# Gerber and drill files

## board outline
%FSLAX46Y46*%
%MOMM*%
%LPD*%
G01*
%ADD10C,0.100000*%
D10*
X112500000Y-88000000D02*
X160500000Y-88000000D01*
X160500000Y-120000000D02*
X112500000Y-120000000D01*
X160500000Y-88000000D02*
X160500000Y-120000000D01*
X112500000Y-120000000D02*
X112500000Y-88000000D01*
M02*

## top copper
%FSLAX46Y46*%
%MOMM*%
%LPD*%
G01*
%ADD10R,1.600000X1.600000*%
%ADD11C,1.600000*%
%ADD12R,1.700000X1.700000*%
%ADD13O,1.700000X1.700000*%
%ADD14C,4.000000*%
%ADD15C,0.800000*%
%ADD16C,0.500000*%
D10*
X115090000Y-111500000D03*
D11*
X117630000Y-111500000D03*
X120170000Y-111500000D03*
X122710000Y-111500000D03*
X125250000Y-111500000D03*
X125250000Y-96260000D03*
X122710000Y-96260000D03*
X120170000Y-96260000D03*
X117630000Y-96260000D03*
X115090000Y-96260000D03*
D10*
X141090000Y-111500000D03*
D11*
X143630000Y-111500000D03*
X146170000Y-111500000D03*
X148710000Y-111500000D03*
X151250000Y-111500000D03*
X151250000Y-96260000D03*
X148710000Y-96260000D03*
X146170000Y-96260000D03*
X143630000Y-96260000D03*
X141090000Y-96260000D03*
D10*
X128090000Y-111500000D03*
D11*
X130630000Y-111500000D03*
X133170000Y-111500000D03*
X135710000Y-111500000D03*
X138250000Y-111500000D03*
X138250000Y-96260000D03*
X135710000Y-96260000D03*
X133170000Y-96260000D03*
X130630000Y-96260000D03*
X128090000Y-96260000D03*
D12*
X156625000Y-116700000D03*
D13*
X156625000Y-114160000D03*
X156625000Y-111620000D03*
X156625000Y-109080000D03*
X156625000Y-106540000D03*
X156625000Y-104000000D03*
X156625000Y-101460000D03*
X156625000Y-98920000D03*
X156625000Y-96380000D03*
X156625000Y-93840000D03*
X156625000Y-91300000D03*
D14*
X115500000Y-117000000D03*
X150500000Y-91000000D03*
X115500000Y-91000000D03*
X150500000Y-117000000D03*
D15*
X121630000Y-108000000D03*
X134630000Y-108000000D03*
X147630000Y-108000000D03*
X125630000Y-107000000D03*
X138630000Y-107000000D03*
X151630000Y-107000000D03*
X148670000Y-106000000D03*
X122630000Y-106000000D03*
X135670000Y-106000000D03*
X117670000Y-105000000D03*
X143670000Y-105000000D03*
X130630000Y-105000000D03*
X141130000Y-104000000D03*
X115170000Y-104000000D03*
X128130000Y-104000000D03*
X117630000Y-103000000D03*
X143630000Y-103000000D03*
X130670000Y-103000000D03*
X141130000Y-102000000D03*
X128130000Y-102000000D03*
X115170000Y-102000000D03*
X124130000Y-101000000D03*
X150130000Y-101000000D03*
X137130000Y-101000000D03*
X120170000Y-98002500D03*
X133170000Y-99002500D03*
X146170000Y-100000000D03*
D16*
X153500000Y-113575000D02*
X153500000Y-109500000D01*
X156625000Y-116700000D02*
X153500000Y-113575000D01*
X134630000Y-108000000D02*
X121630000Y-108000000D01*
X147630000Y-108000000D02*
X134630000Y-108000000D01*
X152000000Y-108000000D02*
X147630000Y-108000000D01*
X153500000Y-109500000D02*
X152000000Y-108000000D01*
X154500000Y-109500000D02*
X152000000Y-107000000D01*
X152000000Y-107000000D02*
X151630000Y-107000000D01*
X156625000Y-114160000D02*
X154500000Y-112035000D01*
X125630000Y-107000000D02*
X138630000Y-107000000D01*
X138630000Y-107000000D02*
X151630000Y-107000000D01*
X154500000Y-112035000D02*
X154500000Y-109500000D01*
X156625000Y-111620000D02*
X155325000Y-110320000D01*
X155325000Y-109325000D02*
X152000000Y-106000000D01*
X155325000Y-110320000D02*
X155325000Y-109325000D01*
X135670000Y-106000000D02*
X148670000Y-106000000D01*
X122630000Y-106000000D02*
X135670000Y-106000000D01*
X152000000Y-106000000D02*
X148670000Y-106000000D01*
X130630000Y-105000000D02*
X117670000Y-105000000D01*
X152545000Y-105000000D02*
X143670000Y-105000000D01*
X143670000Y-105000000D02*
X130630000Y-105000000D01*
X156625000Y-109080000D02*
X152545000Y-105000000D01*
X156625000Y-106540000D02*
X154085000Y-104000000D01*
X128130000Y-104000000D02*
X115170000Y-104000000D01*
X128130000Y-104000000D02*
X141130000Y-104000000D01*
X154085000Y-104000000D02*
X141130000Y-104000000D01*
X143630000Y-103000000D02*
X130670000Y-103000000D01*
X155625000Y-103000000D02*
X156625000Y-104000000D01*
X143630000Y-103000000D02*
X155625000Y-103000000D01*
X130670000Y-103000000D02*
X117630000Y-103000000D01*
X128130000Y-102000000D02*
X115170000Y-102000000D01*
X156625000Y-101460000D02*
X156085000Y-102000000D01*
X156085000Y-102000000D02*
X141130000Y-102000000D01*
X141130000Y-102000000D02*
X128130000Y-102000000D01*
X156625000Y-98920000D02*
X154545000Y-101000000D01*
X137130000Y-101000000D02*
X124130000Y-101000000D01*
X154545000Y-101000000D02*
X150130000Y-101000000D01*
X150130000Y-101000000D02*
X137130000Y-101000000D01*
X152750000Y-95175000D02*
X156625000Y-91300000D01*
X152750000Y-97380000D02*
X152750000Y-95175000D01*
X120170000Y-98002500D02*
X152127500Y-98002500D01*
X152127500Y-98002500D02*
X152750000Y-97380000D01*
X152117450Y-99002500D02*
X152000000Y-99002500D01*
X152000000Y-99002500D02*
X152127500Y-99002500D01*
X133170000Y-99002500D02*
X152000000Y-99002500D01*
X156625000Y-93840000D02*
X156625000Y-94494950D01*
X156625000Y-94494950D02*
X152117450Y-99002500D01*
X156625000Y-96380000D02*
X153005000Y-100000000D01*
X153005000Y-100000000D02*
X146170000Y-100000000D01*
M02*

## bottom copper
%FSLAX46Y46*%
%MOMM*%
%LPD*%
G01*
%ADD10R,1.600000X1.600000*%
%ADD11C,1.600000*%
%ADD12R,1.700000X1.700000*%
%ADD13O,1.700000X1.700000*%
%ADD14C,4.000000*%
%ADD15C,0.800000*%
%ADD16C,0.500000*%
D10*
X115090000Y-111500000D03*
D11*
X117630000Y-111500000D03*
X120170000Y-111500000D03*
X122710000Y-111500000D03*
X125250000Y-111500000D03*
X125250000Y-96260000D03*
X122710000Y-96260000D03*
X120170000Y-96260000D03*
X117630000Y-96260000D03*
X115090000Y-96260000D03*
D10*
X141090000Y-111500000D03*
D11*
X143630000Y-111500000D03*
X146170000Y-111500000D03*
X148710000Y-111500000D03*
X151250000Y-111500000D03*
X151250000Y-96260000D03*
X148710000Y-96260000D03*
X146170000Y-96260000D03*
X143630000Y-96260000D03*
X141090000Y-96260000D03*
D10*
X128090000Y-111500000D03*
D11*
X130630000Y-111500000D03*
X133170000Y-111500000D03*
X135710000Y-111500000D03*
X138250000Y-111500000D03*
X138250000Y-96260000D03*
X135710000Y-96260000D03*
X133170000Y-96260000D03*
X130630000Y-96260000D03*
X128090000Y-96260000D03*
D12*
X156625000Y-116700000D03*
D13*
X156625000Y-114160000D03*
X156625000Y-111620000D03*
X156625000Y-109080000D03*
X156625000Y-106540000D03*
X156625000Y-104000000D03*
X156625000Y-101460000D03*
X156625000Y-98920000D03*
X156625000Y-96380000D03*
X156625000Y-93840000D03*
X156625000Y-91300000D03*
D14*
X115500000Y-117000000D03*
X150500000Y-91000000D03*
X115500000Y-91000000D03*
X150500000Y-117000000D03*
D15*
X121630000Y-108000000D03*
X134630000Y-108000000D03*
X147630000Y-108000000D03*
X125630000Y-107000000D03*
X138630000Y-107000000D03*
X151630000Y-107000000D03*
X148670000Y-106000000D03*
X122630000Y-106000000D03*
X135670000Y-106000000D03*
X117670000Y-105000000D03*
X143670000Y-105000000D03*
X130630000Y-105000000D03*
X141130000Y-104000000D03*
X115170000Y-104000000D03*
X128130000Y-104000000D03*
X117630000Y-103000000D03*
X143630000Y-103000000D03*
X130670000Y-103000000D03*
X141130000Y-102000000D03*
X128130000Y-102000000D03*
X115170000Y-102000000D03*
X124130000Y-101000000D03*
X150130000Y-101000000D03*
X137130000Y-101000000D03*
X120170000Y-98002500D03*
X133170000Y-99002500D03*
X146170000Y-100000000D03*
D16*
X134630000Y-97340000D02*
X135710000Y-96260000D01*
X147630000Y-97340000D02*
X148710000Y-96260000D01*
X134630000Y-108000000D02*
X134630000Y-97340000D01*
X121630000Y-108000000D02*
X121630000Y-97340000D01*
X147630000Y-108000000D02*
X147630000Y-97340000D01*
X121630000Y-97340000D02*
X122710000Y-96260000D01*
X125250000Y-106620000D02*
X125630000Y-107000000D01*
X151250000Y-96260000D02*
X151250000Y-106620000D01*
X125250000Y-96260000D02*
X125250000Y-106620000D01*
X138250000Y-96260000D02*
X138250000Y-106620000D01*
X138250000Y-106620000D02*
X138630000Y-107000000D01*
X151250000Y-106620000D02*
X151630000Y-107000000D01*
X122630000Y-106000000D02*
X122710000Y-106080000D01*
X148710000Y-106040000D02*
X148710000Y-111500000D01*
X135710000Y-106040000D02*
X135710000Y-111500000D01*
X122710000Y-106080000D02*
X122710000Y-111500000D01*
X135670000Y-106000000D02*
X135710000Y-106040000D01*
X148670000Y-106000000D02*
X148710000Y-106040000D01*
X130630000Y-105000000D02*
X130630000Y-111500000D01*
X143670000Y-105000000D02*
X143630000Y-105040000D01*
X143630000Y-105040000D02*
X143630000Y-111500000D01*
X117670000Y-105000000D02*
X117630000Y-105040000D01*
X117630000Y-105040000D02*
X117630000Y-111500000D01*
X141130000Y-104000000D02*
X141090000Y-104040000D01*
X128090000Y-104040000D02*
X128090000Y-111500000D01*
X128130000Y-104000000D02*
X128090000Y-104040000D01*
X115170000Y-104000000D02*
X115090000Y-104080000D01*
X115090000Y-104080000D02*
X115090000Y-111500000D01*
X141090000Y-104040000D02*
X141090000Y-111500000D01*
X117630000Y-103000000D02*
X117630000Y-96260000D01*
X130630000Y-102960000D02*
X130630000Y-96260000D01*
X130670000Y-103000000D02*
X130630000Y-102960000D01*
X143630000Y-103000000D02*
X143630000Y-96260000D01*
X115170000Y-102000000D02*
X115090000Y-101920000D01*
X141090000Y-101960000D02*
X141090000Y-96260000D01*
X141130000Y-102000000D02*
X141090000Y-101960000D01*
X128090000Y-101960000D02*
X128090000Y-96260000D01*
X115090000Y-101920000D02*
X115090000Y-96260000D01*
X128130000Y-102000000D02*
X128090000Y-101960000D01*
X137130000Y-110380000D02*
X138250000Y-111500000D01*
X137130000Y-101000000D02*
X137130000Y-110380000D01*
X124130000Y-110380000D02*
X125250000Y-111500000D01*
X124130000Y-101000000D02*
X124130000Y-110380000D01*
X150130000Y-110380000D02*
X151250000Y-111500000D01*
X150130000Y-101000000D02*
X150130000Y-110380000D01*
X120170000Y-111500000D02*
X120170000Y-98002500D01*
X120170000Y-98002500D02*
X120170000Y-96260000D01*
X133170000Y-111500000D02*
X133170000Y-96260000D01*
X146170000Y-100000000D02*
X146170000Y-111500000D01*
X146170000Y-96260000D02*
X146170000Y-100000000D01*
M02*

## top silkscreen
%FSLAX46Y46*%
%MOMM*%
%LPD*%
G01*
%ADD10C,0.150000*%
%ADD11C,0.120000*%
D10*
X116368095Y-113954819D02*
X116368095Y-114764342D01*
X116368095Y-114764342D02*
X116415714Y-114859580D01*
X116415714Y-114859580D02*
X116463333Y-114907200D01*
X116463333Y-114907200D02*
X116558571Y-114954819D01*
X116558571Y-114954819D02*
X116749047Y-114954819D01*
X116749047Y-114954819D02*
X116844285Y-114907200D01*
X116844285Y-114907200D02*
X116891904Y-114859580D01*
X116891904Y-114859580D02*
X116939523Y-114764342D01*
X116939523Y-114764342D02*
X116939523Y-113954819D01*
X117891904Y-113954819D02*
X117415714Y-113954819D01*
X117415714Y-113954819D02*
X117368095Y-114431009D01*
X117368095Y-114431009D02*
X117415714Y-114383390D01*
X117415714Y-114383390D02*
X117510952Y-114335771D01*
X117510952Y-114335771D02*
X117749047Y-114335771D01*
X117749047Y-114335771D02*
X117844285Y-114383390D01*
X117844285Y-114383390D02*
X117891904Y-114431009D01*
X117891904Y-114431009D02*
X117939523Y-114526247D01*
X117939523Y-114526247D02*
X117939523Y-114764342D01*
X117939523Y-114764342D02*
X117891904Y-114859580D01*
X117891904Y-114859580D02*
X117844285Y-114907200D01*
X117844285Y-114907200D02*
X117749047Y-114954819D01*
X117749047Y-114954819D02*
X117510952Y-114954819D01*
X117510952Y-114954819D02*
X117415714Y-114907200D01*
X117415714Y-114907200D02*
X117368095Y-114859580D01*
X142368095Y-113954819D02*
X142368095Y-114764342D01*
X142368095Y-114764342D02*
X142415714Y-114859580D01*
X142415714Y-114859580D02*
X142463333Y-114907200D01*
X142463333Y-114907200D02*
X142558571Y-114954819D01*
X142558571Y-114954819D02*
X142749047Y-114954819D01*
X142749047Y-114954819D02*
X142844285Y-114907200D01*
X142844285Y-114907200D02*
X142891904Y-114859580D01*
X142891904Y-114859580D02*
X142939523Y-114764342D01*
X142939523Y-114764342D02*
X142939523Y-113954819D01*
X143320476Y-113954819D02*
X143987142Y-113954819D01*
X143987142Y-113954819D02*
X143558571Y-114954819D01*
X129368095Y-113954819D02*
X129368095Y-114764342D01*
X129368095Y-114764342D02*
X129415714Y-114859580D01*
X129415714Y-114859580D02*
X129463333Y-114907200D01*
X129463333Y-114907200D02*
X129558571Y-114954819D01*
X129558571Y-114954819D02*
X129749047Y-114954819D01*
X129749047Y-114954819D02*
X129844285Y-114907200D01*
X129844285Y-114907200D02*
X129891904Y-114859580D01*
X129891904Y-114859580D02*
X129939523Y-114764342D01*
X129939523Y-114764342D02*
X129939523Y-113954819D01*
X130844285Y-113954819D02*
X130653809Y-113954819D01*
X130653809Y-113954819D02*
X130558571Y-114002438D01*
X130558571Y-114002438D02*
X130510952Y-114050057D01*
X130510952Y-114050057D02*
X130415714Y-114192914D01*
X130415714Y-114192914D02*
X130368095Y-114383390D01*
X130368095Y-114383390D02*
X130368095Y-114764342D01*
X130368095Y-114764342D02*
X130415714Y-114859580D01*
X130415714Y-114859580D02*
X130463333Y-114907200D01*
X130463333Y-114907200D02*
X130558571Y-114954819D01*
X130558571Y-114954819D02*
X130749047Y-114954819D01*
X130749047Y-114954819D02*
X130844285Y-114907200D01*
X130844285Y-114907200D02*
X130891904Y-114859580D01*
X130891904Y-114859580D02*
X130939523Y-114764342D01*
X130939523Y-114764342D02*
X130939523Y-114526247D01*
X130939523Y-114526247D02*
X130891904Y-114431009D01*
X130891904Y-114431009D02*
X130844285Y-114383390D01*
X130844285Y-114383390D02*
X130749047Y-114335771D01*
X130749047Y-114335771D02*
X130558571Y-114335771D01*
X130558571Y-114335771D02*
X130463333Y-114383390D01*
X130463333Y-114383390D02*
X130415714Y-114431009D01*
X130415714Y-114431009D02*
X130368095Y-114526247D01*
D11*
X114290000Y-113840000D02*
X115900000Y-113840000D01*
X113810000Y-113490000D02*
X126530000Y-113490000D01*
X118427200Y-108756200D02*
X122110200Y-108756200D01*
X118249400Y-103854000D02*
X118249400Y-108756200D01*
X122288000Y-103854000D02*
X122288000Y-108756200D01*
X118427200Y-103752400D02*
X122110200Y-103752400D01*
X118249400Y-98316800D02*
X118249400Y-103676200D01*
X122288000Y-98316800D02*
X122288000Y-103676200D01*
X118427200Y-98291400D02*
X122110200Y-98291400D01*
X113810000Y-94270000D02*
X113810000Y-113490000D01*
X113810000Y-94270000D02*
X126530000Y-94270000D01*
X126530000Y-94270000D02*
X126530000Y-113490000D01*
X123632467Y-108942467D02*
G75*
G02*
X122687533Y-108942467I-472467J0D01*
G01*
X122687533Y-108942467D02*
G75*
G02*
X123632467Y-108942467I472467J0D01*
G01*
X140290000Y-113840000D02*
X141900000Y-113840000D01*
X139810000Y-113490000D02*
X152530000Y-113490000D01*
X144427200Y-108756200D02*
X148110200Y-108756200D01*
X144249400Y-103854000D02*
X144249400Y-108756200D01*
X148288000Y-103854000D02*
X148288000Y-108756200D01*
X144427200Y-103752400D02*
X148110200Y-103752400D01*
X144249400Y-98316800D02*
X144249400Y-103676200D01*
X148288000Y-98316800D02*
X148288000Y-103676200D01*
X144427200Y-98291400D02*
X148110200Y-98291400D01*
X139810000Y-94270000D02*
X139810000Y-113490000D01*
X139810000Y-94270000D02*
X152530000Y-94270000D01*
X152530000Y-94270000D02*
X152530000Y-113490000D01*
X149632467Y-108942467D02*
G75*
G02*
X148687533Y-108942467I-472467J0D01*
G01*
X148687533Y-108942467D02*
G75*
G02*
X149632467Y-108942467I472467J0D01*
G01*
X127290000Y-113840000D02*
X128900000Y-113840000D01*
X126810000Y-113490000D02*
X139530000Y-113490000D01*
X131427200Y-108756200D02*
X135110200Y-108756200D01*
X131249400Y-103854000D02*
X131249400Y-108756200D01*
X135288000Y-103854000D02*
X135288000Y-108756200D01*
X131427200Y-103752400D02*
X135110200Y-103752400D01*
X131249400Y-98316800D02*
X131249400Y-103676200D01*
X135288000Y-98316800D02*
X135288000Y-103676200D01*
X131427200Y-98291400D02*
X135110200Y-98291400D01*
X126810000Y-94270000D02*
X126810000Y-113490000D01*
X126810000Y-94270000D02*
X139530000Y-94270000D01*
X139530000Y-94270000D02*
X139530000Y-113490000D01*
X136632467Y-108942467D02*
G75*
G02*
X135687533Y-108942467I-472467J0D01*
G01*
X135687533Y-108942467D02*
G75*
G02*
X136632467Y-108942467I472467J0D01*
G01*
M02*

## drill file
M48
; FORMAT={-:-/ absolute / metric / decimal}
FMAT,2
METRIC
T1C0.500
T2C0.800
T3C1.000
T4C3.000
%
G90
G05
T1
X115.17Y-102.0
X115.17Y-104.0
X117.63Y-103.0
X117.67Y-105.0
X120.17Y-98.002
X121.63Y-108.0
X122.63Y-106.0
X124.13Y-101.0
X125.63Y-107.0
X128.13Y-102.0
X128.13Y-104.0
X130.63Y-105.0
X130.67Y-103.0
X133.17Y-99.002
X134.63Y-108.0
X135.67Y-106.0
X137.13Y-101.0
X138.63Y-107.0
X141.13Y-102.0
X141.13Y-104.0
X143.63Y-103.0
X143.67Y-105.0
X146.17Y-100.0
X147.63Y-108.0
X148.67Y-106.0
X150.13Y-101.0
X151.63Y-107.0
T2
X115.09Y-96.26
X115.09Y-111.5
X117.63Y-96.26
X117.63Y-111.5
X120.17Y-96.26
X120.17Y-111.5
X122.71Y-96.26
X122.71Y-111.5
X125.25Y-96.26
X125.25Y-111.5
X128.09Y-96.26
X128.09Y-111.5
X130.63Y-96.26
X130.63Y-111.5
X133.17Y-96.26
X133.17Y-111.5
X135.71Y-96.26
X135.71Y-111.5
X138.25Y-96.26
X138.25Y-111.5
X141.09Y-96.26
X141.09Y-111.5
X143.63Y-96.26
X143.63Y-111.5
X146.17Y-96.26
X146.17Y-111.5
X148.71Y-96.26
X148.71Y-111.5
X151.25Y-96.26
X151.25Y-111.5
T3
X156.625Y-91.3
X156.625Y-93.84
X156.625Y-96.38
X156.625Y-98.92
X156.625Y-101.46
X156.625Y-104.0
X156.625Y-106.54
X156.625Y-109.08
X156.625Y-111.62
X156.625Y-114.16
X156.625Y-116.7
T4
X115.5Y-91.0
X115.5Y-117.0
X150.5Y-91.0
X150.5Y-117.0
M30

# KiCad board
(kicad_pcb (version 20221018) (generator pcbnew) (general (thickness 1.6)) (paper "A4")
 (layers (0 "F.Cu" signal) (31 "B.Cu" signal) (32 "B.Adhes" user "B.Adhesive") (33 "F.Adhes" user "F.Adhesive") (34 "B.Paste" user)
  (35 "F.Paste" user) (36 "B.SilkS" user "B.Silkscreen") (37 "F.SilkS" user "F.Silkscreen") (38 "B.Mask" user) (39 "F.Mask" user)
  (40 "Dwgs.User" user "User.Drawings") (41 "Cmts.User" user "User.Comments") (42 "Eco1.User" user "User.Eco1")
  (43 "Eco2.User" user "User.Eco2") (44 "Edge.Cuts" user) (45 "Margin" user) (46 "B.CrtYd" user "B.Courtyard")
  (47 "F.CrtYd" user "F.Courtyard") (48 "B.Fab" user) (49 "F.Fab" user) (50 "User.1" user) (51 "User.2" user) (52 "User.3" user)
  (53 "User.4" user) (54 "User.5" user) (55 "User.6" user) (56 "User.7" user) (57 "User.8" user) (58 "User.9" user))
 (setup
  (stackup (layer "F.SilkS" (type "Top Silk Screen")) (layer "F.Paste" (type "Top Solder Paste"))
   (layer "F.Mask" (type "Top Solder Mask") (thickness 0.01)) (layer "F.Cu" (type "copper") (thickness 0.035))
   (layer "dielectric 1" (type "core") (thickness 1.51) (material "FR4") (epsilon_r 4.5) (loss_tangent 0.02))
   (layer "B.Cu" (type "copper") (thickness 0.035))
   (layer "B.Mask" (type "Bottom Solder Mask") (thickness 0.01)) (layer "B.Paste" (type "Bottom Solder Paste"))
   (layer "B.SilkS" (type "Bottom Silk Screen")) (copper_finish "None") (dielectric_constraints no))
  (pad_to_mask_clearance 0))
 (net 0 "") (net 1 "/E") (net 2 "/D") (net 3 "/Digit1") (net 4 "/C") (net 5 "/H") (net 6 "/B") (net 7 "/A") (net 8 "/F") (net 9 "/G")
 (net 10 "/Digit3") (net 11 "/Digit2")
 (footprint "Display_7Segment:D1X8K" (layer "F.Cu") (at 115.09 111.5 90)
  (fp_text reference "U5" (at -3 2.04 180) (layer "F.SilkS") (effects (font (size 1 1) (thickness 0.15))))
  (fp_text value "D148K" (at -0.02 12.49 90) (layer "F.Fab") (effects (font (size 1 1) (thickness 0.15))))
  (fp_line (start -2.34 -0.8) (end -2.34 0.81) (stroke (width 0.12) (type solid)) (layer "F.SilkS"))
  (fp_line (start -1.99 -1.28) (end -1.99 11.44) (stroke (width 0.12) (type solid)) (layer "F.SilkS"))
  (fp_line (start 2.7438 3.3372) (end 2.7438 7.0202) (stroke (width 0.12) (type solid)) (layer "F.SilkS"))
  (fp_line (start 7.646 3.1594) (end 2.7438 3.1594) (stroke (width 0.12) (type solid)) (layer "F.SilkS"))
  (fp_line (start 7.646 7.198) (end 2.7438 7.198) (stroke (width 0.12) (type solid)) (layer "F.SilkS"))
  (fp_line (start 7.7476 3.3372) (end 7.7476 7.0202) (stroke (width 0.12) (type solid)) (layer "F.SilkS"))
  (fp_line (start 13.1832 3.1594) (end 7.8238 3.1594) (stroke (width 0.12) (type solid)) (layer "F.SilkS"))
  (fp_line (start 13.1832 7.198) (end 7.8238 7.198) (stroke (width 0.12) (type solid)) (layer "F.SilkS"))
  (fp_line (start 13.2086 3.3372) (end 13.2086 7.0202) (stroke (width 0.12) (type solid)) (layer "F.SilkS"))
  (fp_line (start 17.23 -1.28) (end -1.99 -1.28) (stroke (width 0.12) (type solid)) (layer "F.SilkS"))
  (fp_line (start 17.23 -1.28) (end 17.23 11.44) (stroke (width 0.12) (type solid)) (layer "F.SilkS"))
  (fp_line (start 17.23 11.44) (end -1.99 11.44) (stroke (width 0.12) (type solid)) (layer "F.SilkS"))
  (fp_circle (center 2.557533 8.07) (end 2.836933 7.689) (stroke (width 0.12) (type solid)) (fill none) (layer "F.SilkS"))
  (pad "1" thru_hole rect (at 0 0) (size 1.6 1.6) (drill 0.8) (layers "*.Cu" "*.Mask") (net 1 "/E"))
  (pad "2" thru_hole circle (at 0 2.54) (size 1.6 1.6) (drill 0.8) (layers "*.Cu" "*.Mask") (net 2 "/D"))
  (pad "3" thru_hole circle (at 0 5.08) (size 1.6 1.6) (drill 0.8) (layers "*.Cu" "*.Mask") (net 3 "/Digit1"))
  (pad "4" thru_hole circle (at 0 7.62) (size 1.6 1.6) (drill 0.8) (layers "*.Cu" "*.Mask") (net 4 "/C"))
  (pad "5" thru_hole circle (at 0 10.16) (size 1.6 1.6) (drill 0.8) (layers "*.Cu" "*.Mask") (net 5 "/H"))
  (pad "6" thru_hole circle (at 15.24 10.16) (size 1.6 1.6) (drill 0.8) (layers "*.Cu" "*.Mask") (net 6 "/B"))
  (pad "7" thru_hole circle (at 15.24 7.62) (size 1.6 1.6) (drill 0.8) (layers "*.Cu" "*.Mask") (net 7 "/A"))
  (pad "8" thru_hole circle (at 15.24 5.08) (size 1.6 1.6) (drill 0.8) (layers "*.Cu" "*.Mask") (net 3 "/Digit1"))
  (pad "9" thru_hole circle (at 15.24 2.54) (size 1.6 1.6) (drill 0.8) (layers "*.Cu" "*.Mask") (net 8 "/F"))
  (pad "10" thru_hole circle (at 15.24 0) (size 1.6 1.6) (drill 0.8) (layers "*.Cu" "*.Mask") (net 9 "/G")))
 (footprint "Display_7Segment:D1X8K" (layer "F.Cu") (at 141.09 111.5 90)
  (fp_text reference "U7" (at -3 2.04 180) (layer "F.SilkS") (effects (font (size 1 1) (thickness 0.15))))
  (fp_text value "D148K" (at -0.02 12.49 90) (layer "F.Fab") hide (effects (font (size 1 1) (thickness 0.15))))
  (fp_line (start -2.34 -0.8) (end -2.34 0.81) (stroke (width 0.12) (type solid)) (layer "F.SilkS"))
  (fp_line (start -1.99 -1.28) (end -1.99 11.44) (stroke (width 0.12) (type solid)) (layer "F.SilkS"))
  (fp_line (start 2.7438 3.3372) (end 2.7438 7.0202) (stroke (width 0.12) (type solid)) (layer "F.SilkS"))
  (fp_line (start 7.646 3.1594) (end 2.7438 3.1594) (stroke (width 0.12) (type solid)) (layer "F.SilkS"))
  (fp_line (start 7.646 7.198) (end 2.7438 7.198) (stroke (width 0.12) (type solid)) (layer "F.SilkS"))
  (fp_line (start 7.7476 3.3372) (end 7.7476 7.0202) (stroke (width 0.12) (type solid)) (layer "F.SilkS"))
  (fp_line (start 13.1832 3.1594) (end 7.8238 3.1594) (stroke (width 0.12) (type solid)) (layer "F.SilkS"))
  (fp_line (start 13.1832 7.198) (end 7.8238 7.198) (stroke (width 0.12) (type solid)) (layer "F.SilkS"))
  (fp_line (start 13.2086 3.3372) (end 13.2086 7.0202) (stroke (width 0.12) (type solid)) (layer "F.SilkS"))
  (fp_line (start 17.23 -1.28) (end -1.99 -1.28) (stroke (width 0.12) (type solid)) (layer "F.SilkS"))
  (fp_line (start 17.23 -1.28) (end 17.23 11.44) (stroke (width 0.12) (type solid)) (layer "F.SilkS"))
  (fp_line (start 17.23 11.44) (end -1.99 11.44) (stroke (width 0.12) (type solid)) (layer "F.SilkS"))
  (fp_circle (center 2.557533 8.07) (end 2.836933 7.689) (stroke (width 0.12) (type solid)) (fill none) (layer "F.SilkS"))
  (pad "1" thru_hole rect (at 0 0) (size 1.6 1.6) (drill 0.8) (layers "*.Cu" "*.Mask") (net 1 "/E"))
  (pad "2" thru_hole circle (at 0 2.54) (size 1.6 1.6) (drill 0.8) (layers "*.Cu" "*.Mask") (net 2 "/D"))
  (pad "3" thru_hole circle (at 0 5.08) (size 1.6 1.6) (drill 0.8) (layers "*.Cu" "*.Mask") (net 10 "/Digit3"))
  (pad "4" thru_hole circle (at 0 7.62) (size 1.6 1.6) (drill 0.8) (layers "*.Cu" "*.Mask") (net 4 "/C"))
  (pad "5" thru_hole circle (at 0 10.16) (size 1.6 1.6) (drill 0.8) (layers "*.Cu" "*.Mask") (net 5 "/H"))
  (pad "6" thru_hole circle (at 15.24 10.16) (size 1.6 1.6) (drill 0.8) (layers "*.Cu" "*.Mask") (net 6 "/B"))
  (pad "7" thru_hole circle (at 15.24 7.62) (size 1.6 1.6) (drill 0.8) (layers "*.Cu" "*.Mask") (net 7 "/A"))
  (pad "8" thru_hole circle (at 15.24 5.08) (size 1.6 1.6) (drill 0.8) (layers "*.Cu" "*.Mask") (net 10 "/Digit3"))
  (pad "9" thru_hole circle (at 15.24 2.54) (size 1.6 1.6) (drill 0.8) (layers "*.Cu" "*.Mask") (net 8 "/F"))
  (pad "10" thru_hole circle (at 15.24 0) (size 1.6 1.6) (drill 0.8) (layers "*.Cu" "*.Mask") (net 9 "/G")))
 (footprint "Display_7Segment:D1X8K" (layer "F.Cu") (at 128.09 111.5 90)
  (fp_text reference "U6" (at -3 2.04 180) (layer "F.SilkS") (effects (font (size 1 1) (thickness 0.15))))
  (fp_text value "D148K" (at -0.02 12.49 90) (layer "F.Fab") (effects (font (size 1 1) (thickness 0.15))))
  (fp_line (start -2.34 -0.8) (end -2.34 0.81) (stroke (width 0.12) (type solid)) (layer "F.SilkS"))
  (fp_line (start -1.99 -1.28) (end -1.99 11.44) (stroke (width 0.12) (type solid)) (layer "F.SilkS"))
  (fp_line (start 2.7438 3.3372) (end 2.7438 7.0202) (stroke (width 0.12) (type solid)) (layer "F.SilkS"))
  (fp_line (start 7.646 3.1594) (end 2.7438 3.1594) (stroke (width 0.12) (type solid)) (layer "F.SilkS"))
  (fp_line (start 7.646 7.198) (end 2.7438 7.198) (stroke (width 0.12) (type solid)) (layer "F.SilkS"))
  (fp_line (start 7.7476 3.3372) (end 7.7476 7.0202) (stroke (width 0.12) (type solid)) (layer "F.SilkS"))
  (fp_line (start 13.1832 3.1594) (end 7.8238 3.1594) (stroke (width 0.12) (type solid)) (layer "F.SilkS"))
  (fp_line (start 13.1832 7.198) (end 7.8238 7.198) (stroke (width 0.12) (type solid)) (layer "F.SilkS"))
  (fp_line (start 13.2086 3.3372) (end 13.2086 7.0202) (stroke (width 0.12) (type solid)) (layer "F.SilkS"))
  (fp_line (start 17.23 -1.28) (end -1.99 -1.28) (stroke (width 0.12) (type solid)) (layer "F.SilkS"))
  (fp_line (start 17.23 -1.28) (end 17.23 11.44) (stroke (width 0.12) (type solid)) (layer "F.SilkS"))
  (fp_line (start 17.23 11.44) (end -1.99 11.44) (stroke (width 0.12) (type solid)) (layer "F.SilkS"))
  (fp_circle (center 2.557533 8.07) (end 2.836933 7.689) (stroke (width 0.12) (type solid)) (fill none) (layer "F.SilkS"))
  (pad "1" thru_hole rect (at 0 0) (size 1.6 1.6) (drill 0.8) (layers "*.Cu" "*.Mask") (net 1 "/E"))
  (pad "2" thru_hole circle (at 0 2.54) (size 1.6 1.6) (drill 0.8) (layers "*.Cu" "*.Mask") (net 2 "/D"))
  (pad "3" thru_hole circle (at 0 5.08) (size 1.6 1.6) (drill 0.8) (layers "*.Cu" "*.Mask") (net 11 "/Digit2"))
  (pad "4" thru_hole circle (at 0 7.62) (size 1.6 1.6) (drill 0.8) (layers "*.Cu" "*.Mask") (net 4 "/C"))
  (pad "5" thru_hole circle (at 0 10.16) (size 1.6 1.6) (drill 0.8) (layers "*.Cu" "*.Mask") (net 5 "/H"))
  (pad "6" thru_hole circle (at 15.24 10.16) (size 1.6 1.6) (drill 0.8) (layers "*.Cu" "*.Mask") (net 6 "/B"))
  (pad "7" thru_hole circle (at 15.24 7.62) (size 1.6 1.6) (drill 0.8) (layers "*.Cu" "*.Mask") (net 7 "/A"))
  (pad "8" thru_hole circle (at 15.24 5.08) (size 1.6 1.6) (drill 0.8) (layers "*.Cu" "*.Mask") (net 11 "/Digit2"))
  (pad "9" thru_hole circle (at 15.24 2.54) (size 1.6 1.6) (drill 0.8) (layers "*.Cu" "*.Mask") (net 8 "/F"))
  (pad "10" thru_hole circle (at 15.24 0) (size 1.6 1.6) (drill 0.8) (layers "*.Cu" "*.Mask") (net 9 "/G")))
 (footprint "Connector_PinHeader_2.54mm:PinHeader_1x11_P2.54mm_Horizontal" (layer "B.Cu") (at 156.625 116.7)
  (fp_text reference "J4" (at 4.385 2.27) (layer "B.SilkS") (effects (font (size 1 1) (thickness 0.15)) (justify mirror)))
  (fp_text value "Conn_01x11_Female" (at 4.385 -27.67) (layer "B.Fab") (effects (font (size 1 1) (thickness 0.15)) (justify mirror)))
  (pad "1" thru_hole rect (at 0 0) (size 1.7 1.7) (drill 1) (layers "*.Cu" "*.Mask") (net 7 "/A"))
  (pad "2" thru_hole oval (at 0 -2.54) (size 1.7 1.7) (drill 1) (layers "*.Cu" "*.Mask") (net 6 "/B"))
  (pad "3" thru_hole oval (at 0 -5.08) (size 1.7 1.7) (drill 1) (layers "*.Cu" "*.Mask") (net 4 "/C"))
  (pad "4" thru_hole oval (at 0 -7.62) (size 1.7 1.7) (drill 1) (layers "*.Cu" "*.Mask") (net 2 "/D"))
  (pad "5" thru_hole oval (at 0 -10.16) (size 1.7 1.7) (drill 1) (layers "*.Cu" "*.Mask") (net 1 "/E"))
  (pad "6" thru_hole oval (at 0 -12.7) (size 1.7 1.7) (drill 1) (layers "*.Cu" "*.Mask") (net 8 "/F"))
  (pad "7" thru_hole oval (at 0 -15.24) (size 1.7 1.7) (drill 1) (layers "*.Cu" "*.Mask") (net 9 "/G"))
  (pad "8" thru_hole oval (at 0 -17.78) (size 1.7 1.7) (drill 1) (layers "*.Cu" "*.Mask") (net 5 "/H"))
  (pad "9" thru_hole oval (at 0 -20.32) (size 1.7 1.7) (drill 1) (layers "*.Cu" "*.Mask") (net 10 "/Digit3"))
  (pad "10" thru_hole oval (at 0 -22.86) (size 1.7 1.7) (drill 1) (layers "*.Cu" "*.Mask") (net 11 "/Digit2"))
  (pad "11" thru_hole oval (at 0 -25.4) (size 1.7 1.7) (drill 1) (layers "*.Cu" "*.Mask") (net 3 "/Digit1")))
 (gr_line (start 112.5 88) (end 160.5 88) (stroke (width 0.1) (type solid)) (layer "Edge.Cuts"))
 (gr_line (start 160.5 120) (end 112.5 120) (stroke (width 0.1) (type solid)) (layer "Edge.Cuts"))
 (gr_line (start 160.5 88) (end 160.5 120) (stroke (width 0.1) (type solid)) (layer "Edge.Cuts"))
 (gr_line (start 112.5 120) (end 112.5 88) (stroke (width 0.1) (type solid)) (layer "Edge.Cuts"))
 (via (at 115.5 117) (size 4) (drill 3) (layers "F.Cu" "B.Cu") (free) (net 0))
 (via (at 150.5 91) (size 4) (drill 3) (layers "F.Cu" "B.Cu") (free) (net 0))
 (via (at 115.5 91) (size 4) (drill 3) (layers "F.Cu" "B.Cu") (free) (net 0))
 (via (at 150.5 117) (size 4) (drill 3) (layers "F.Cu" "B.Cu") (free) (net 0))
 (segment (start 153.5 113.575) (end 153.5 109.5) (width 0.5) (layer "F.Cu") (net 7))
 (segment (start 156.625 116.7) (end 153.5 113.575) (width 0.5) (layer "F.Cu") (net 7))
 (segment (start 134.63 108) (end 121.63 108) (width 0.5) (layer "F.Cu") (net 7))
 (segment (start 147.63 108) (end 134.63 108) (width 0.5) (layer "F.Cu") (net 7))
 (segment (start 152 108) (end 147.63 108) (width 0.5) (layer "F.Cu") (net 7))
 (segment (start 153.5 109.5) (end 152 108) (width 0.5) (layer "F.Cu") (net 7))
 (via (at 121.63 108) (size 0.8) (drill 0.5) (layers "F.Cu" "B.Cu") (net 7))
 (via (at 134.63 108) (size 0.8) (drill 0.5) (layers "F.Cu" "B.Cu") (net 7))
 (via (at 147.63 108) (size 0.8) (drill 0.5) (layers "F.Cu" "B.Cu") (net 7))
 (segment (start 134.63 97.34) (end 135.71 96.26) (width 0.5) (layer "B.Cu") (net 7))
 (segment (start 147.63 97.34) (end 148.71 96.26) (width 0.5) (layer "B.Cu") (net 7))
 (segment (start 134.63 108) (end 134.63 97.34) (width 0.5) (layer "B.Cu") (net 7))
 (segment (start 121.63 108) (end 121.63 97.34) (width 0.5) (layer "B.Cu") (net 7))
 (segment (start 147.63 108) (end 147.63 97.34) (width 0.5) (layer "B.Cu") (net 7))
 (segment (start 121.63 97.34) (end 122.71 96.26) (width 0.5) (layer "B.Cu") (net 7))
 (segment (start 154.5 109.5) (end 152 107) (width 0.5) (layer "F.Cu") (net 6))
 (segment (start 152 107) (end 151.63 107) (width 0.5) (layer "F.Cu") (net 6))
 (segment (start 156.625 114.16) (end 154.5 112.035) (width 0.5) (layer "F.Cu") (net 6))
 (segment (start 125.63 107) (end 138.63 107) (width 0.5) (layer "F.Cu") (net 6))
 (segment (start 138.63 107) (end 151.63 107) (width 0.5) (layer "F.Cu") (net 6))
 (segment (start 154.5 112.035) (end 154.5 109.5) (width 0.5) (layer "F.Cu") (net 6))
 (via (at 125.63 107) (size 0.8) (drill 0.5) (layers "F.Cu" "B.Cu") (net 6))
 (via (at 138.63 107) (size 0.8) (drill 0.5) (layers "F.Cu" "B.Cu") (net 6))
 (via (at 151.63 107) (size 0.8) (drill 0.5) (layers "F.Cu" "B.Cu") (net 6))
 (segment (start 125.25 106.62) (end 125.63 107) (width 0.5) (layer "B.Cu") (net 6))
 (segment (start 151.25 96.26) (end 151.25 106.62) (width 0.5) (layer "B.Cu") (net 6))
 (segment (start 125.25 96.26) (end 125.25 106.62) (width 0.5) (layer "B.Cu") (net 6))
 (segment (start 138.25 96.26) (end 138.25 106.62) (width 0.5) (layer "B.Cu") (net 6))
 (segment (start 138.25 106.62) (end 138.63 107) (width 0.5) (layer "B.Cu") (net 6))
 (segment (start 151.25 106.62) (end 151.63 107) (width 0.5) (layer "B.Cu") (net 6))
 (segment (start 156.625 111.62) (end 155.325 110.32) (width 0.5) (layer "F.Cu") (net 4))
 (segment (start 155.325 109.325) (end 152 106) (width 0.5) (layer "F.Cu") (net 4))
 (segment (start 155.325 110.32) (end 155.325 109.325) (width 0.5) (layer "F.Cu") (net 4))
 (segment (start 135.67 106) (end 148.67 106) (width 0.5) (layer "F.Cu") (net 4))
 (segment (start 122.63 106) (end 135.67 106) (width 0.5) (layer "F.Cu") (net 4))
 (segment (start 152 106) (end 148.67 106) (width 0.5) (layer "F.Cu") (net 4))
 (via (at 148.67 106) (size 0.8) (drill 0.5) (layers "F.Cu" "B.Cu") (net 4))
 (via (at 122.63 106) (size 0.8) (drill 0.5) (layers "F.Cu" "B.Cu") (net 4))
 (via (at 135.67 106) (size 0.8) (drill 0.5) (layers "F.Cu" "B.Cu") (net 4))
 (segment (start 122.63 106) (end 122.71 106.08) (width 0.5) (layer "B.Cu") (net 4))
 (segment (start 148.71 106.04) (end 148.71 111.5) (width 0.5) (layer "B.Cu") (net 4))
 (segment (start 135.71 106.04) (end 135.71 111.5) (width 0.5) (layer "B.Cu") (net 4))
 (segment (start 122.71 106.08) (end 122.71 111.5) (width 0.5) (layer "B.Cu") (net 4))
 (segment (start 135.67 106) (end 135.71 106.04) (width 0.5) (layer "B.Cu") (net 4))
 (segment (start 148.67 106) (end 148.71 106.04) (width 0.5) (layer "B.Cu") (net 4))
 (segment (start 130.63 105) (end 117.67 105) (width 0.5) (layer "F.Cu") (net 2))
 (segment (start 152.545 105) (end 143.67 105) (width 0.5) (layer "F.Cu") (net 2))
 (segment (start 143.67 105) (end 130.63 105) (width 0.5) (layer "F.Cu") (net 2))
 (segment (start 156.625 109.08) (end 152.545 105) (width 0.5) (layer "F.Cu") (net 2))
 (via (at 117.67 105) (size 0.8) (drill 0.5) (layers "F.Cu" "B.Cu") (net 2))
 (via (at 143.67 105) (size 0.8) (drill 0.5) (layers "F.Cu" "B.Cu") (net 2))
 (via (at 130.63 105) (size 0.8) (drill 0.5) (layers "F.Cu" "B.Cu") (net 2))
 (segment (start 130.63 105) (end 130.63 111.5) (width 0.5) (layer "B.Cu") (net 2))
 (segment (start 143.67 105) (end 143.63 105.04) (width 0.5) (layer "B.Cu") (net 2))
 (segment (start 143.63 105.04) (end 143.63 111.5) (width 0.5) (layer "B.Cu") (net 2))
 (segment (start 117.67 105) (end 117.63 105.04) (width 0.5) (layer "B.Cu") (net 2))
 (segment (start 117.63 105.04) (end 117.63 111.5) (width 0.5) (layer "B.Cu") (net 2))
 (segment (start 156.625 106.54) (end 154.085 104) (width 0.5) (layer "F.Cu") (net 1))
 (segment (start 128.13 104) (end 115.17 104) (width 0.5) (layer "F.Cu") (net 1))
 (segment (start 128.13 104) (end 141.13 104) (width 0.5) (layer "F.Cu") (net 1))
 (segment (start 154.085 104) (end 141.13 104) (width 0.5) (layer "F.Cu") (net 1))
 (via (at 141.13 104) (size 0.8) (drill 0.5) (layers "F.Cu" "B.Cu") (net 1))
 (via (at 115.17 104) (size 0.8) (drill 0.5) (layers "F.Cu" "B.Cu") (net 1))
 (via (at 128.13 104) (size 0.8) (drill 0.5) (layers "F.Cu" "B.Cu") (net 1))
 (segment (start 141.13 104) (end 141.09 104.04) (width 0.5) (layer "B.Cu") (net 1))
 (segment (start 128.09 104.04) (end 128.09 111.5) (width 0.5) (layer "B.Cu") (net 1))
 (segment (start 128.13 104) (end 128.09 104.04) (width 0.5) (layer "B.Cu") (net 1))
 (segment (start 115.17 104) (end 115.09 104.08) (width 0.5) (layer "B.Cu") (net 1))
 (segment (start 115.09 104.08) (end 115.09 111.5) (width 0.5) (layer "B.Cu") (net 1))
 (segment (start 141.09 104.04) (end 141.09 111.5) (width 0.5) (layer "B.Cu") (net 1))
 (segment (start 143.63 103) (end 130.67 103) (width 0.5) (layer "F.Cu") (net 8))
 (segment (start 155.625 103) (end 156.625 104) (width 0.5) (layer "F.Cu") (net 8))
 (segment (start 143.63 103) (end 155.625 103) (width 0.5) (layer "F.Cu") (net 8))
 (segment (start 130.67 103) (end 117.63 103) (width 0.5) (layer "F.Cu") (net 8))
 (via (at 117.63 103) (size 0.8) (drill 0.5) (layers "F.Cu" "B.Cu") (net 8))
 (via (at 143.63 103) (size 0.8) (drill 0.5) (layers "F.Cu" "B.Cu") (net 8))
 (via (at 130.67 103) (size 0.8) (drill 0.5) (layers "F.Cu" "B.Cu") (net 8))
 (segment (start 117.63 103) (end 117.63 96.26) (width 0.5) (layer "B.Cu") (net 8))
 (segment (start 130.63 102.96) (end 130.63 96.26) (width 0.5) (layer "B.Cu") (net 8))
 (segment (start 130.67 103) (end 130.63 102.96) (width 0.5) (layer "B.Cu") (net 8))
 (segment (start 143.63 103) (end 143.63 96.26) (width 0.5) (layer "B.Cu") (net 8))
 (segment (start 128.13 102) (end 115.17 102) (width 0.5) (layer "F.Cu") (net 9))
 (segment (start 156.625 101.46) (end 156.085 102) (width 0.5) (layer "F.Cu") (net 9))
 (segment (start 156.085 102) (end 141.13 102) (width 0.5) (layer "F.Cu") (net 9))
 (segment (start 141.13 102) (end 128.13 102) (width 0.5) (layer "F.Cu") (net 9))
 (via (at 141.13 102) (size 0.8) (drill 0.5) (layers "F.Cu" "B.Cu") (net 9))
 (via (at 128.13 102) (size 0.8) (drill 0.5) (layers "F.Cu" "B.Cu") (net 9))
 (via (at 115.17 102) (size 0.8) (drill 0.5) (layers "F.Cu" "B.Cu") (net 9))
 (segment (start 115.17 102) (end 115.09 101.92) (width 0.5) (layer "B.Cu") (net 9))
 (segment (start 141.09 101.96) (end 141.09 96.26) (width 0.5) (layer "B.Cu") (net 9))
 (segment (start 141.13 102) (end 141.09 101.96) (width 0.5) (layer "B.Cu") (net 9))
 (segment (start 128.09 101.96) (end 128.09 96.26) (width 0.5) (layer "B.Cu") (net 9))
 (segment (start 115.09 101.92) (end 115.09 96.26) (width 0.5) (layer "B.Cu") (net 9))
 (segment (start 128.13 102) (end 128.09 101.96) (width 0.5) (layer "B.Cu") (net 9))
 (segment (start 156.625 98.92) (end 154.545 101) (width 0.5) (layer "F.Cu") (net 5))
 (segment (start 137.13 101) (end 124.13 101) (width 0.5) (layer "F.Cu") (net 5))
 (segment (start 154.545 101) (end 150.13 101) (width 0.5) (layer "F.Cu") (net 5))
 (segment (start 150.13 101) (end 137.13 101) (width 0.5) (layer "F.Cu") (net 5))
 (via (at 124.13 101) (size 0.8) (drill 0.5) (layers "F.Cu" "B.Cu") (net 5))
 (via (at 150.13 101) (size 0.8) (drill 0.5) (layers "F.Cu" "B.Cu") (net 5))
 (via (at 137.13 101) (size 0.8) (drill 0.5) (layers "F.Cu" "B.Cu") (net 5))
 (segment (start 137.13 110.38) (end 138.25 111.5) (width 0.5) (layer "B.Cu") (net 5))
 (segment (start 137.13 101) (end 137.13 110.38) (width 0.5) (layer "B.Cu") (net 5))
 (segment (start 124.13 110.38) (end 125.25 111.5) (width 0.5) (layer "B.Cu") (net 5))
 (segment (start 124.13 101) (end 124.13 110.38) (width 0.5) (layer "B.Cu") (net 5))
 (segment (start 150.13 110.38) (end 151.25 111.5) (width 0.5) (layer "B.Cu") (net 5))
 (segment (start 150.13 101) (end 150.13 110.38) (width 0.5) (layer "B.Cu") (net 5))
 (segment (start 152.75 95.175) (end 156.625 91.3) (width 0.5) (layer "F.Cu") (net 3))
 (segment (start 152.75 97.38) (end 152.75 95.175) (width 0.5) (layer "F.Cu") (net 3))
 (segment (start 120.17 98.0025) (end 152.1275 98.0025) (width 0.5) (layer "F.Cu") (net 3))
 (segment (start 152.1275 98.0025) (end 152.75 97.38) (width 0.5) (layer "F.Cu") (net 3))
 (via (at 120.17 98.0025) (size 0.8) (drill 0.5) (layers "F.Cu" "B.Cu") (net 3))
 (segment (start 120.17 111.5) (end 120.17 98.0025) (width 0.5) (layer "B.Cu") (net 3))
 (segment (start 120.17 98.0025) (end 120.17 96.26) (width 0.5) (layer "B.Cu") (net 3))
 (segment (start 152.11745 99.0025) (end 152 99.0025) (width 0.5) (layer "F.Cu") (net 11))
 (segment (start 152 99.0025) (end 152.1275 99.0025) (width 0.5) (layer "F.Cu") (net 11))
 (segment (start 133.17 99.0025) (end 152 99.0025) (width 0.5) (layer "F.Cu") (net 11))
 (segment (start 156.625 93.84) (end 156.625 94.49495) (width 0.5) (layer "F.Cu") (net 11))
 (segment (start 156.625 94.49495) (end 152.11745 99.0025) (width 0.5) (layer "F.Cu") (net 11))
 (via (at 133.17 99.0025) (size 0.8) (drill 0.5) (layers "F.Cu" "B.Cu") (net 11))
 (segment (start 133.17 111.5) (end 133.17 96.26) (width 0.5) (layer "B.Cu") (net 11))
 (segment (start 156.625 96.38) (end 153.005 100) (width 0.5) (layer "F.Cu") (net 10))
 (segment (start 153.005 100) (end 146.17 100) (width 0.5) (layer "F.Cu") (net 10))
 (via (at 146.17 100) (size 0.8) (drill 0.5) (layers "F.Cu" "B.Cu") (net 10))
 (segment (start 146.17 100) (end 146.17 111.5) (width 0.5) (layer "B.Cu") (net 10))
 (segment (start 146.17 96.26) (end 146.17 100) (width 0.5) (layer "B.Cu") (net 10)))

